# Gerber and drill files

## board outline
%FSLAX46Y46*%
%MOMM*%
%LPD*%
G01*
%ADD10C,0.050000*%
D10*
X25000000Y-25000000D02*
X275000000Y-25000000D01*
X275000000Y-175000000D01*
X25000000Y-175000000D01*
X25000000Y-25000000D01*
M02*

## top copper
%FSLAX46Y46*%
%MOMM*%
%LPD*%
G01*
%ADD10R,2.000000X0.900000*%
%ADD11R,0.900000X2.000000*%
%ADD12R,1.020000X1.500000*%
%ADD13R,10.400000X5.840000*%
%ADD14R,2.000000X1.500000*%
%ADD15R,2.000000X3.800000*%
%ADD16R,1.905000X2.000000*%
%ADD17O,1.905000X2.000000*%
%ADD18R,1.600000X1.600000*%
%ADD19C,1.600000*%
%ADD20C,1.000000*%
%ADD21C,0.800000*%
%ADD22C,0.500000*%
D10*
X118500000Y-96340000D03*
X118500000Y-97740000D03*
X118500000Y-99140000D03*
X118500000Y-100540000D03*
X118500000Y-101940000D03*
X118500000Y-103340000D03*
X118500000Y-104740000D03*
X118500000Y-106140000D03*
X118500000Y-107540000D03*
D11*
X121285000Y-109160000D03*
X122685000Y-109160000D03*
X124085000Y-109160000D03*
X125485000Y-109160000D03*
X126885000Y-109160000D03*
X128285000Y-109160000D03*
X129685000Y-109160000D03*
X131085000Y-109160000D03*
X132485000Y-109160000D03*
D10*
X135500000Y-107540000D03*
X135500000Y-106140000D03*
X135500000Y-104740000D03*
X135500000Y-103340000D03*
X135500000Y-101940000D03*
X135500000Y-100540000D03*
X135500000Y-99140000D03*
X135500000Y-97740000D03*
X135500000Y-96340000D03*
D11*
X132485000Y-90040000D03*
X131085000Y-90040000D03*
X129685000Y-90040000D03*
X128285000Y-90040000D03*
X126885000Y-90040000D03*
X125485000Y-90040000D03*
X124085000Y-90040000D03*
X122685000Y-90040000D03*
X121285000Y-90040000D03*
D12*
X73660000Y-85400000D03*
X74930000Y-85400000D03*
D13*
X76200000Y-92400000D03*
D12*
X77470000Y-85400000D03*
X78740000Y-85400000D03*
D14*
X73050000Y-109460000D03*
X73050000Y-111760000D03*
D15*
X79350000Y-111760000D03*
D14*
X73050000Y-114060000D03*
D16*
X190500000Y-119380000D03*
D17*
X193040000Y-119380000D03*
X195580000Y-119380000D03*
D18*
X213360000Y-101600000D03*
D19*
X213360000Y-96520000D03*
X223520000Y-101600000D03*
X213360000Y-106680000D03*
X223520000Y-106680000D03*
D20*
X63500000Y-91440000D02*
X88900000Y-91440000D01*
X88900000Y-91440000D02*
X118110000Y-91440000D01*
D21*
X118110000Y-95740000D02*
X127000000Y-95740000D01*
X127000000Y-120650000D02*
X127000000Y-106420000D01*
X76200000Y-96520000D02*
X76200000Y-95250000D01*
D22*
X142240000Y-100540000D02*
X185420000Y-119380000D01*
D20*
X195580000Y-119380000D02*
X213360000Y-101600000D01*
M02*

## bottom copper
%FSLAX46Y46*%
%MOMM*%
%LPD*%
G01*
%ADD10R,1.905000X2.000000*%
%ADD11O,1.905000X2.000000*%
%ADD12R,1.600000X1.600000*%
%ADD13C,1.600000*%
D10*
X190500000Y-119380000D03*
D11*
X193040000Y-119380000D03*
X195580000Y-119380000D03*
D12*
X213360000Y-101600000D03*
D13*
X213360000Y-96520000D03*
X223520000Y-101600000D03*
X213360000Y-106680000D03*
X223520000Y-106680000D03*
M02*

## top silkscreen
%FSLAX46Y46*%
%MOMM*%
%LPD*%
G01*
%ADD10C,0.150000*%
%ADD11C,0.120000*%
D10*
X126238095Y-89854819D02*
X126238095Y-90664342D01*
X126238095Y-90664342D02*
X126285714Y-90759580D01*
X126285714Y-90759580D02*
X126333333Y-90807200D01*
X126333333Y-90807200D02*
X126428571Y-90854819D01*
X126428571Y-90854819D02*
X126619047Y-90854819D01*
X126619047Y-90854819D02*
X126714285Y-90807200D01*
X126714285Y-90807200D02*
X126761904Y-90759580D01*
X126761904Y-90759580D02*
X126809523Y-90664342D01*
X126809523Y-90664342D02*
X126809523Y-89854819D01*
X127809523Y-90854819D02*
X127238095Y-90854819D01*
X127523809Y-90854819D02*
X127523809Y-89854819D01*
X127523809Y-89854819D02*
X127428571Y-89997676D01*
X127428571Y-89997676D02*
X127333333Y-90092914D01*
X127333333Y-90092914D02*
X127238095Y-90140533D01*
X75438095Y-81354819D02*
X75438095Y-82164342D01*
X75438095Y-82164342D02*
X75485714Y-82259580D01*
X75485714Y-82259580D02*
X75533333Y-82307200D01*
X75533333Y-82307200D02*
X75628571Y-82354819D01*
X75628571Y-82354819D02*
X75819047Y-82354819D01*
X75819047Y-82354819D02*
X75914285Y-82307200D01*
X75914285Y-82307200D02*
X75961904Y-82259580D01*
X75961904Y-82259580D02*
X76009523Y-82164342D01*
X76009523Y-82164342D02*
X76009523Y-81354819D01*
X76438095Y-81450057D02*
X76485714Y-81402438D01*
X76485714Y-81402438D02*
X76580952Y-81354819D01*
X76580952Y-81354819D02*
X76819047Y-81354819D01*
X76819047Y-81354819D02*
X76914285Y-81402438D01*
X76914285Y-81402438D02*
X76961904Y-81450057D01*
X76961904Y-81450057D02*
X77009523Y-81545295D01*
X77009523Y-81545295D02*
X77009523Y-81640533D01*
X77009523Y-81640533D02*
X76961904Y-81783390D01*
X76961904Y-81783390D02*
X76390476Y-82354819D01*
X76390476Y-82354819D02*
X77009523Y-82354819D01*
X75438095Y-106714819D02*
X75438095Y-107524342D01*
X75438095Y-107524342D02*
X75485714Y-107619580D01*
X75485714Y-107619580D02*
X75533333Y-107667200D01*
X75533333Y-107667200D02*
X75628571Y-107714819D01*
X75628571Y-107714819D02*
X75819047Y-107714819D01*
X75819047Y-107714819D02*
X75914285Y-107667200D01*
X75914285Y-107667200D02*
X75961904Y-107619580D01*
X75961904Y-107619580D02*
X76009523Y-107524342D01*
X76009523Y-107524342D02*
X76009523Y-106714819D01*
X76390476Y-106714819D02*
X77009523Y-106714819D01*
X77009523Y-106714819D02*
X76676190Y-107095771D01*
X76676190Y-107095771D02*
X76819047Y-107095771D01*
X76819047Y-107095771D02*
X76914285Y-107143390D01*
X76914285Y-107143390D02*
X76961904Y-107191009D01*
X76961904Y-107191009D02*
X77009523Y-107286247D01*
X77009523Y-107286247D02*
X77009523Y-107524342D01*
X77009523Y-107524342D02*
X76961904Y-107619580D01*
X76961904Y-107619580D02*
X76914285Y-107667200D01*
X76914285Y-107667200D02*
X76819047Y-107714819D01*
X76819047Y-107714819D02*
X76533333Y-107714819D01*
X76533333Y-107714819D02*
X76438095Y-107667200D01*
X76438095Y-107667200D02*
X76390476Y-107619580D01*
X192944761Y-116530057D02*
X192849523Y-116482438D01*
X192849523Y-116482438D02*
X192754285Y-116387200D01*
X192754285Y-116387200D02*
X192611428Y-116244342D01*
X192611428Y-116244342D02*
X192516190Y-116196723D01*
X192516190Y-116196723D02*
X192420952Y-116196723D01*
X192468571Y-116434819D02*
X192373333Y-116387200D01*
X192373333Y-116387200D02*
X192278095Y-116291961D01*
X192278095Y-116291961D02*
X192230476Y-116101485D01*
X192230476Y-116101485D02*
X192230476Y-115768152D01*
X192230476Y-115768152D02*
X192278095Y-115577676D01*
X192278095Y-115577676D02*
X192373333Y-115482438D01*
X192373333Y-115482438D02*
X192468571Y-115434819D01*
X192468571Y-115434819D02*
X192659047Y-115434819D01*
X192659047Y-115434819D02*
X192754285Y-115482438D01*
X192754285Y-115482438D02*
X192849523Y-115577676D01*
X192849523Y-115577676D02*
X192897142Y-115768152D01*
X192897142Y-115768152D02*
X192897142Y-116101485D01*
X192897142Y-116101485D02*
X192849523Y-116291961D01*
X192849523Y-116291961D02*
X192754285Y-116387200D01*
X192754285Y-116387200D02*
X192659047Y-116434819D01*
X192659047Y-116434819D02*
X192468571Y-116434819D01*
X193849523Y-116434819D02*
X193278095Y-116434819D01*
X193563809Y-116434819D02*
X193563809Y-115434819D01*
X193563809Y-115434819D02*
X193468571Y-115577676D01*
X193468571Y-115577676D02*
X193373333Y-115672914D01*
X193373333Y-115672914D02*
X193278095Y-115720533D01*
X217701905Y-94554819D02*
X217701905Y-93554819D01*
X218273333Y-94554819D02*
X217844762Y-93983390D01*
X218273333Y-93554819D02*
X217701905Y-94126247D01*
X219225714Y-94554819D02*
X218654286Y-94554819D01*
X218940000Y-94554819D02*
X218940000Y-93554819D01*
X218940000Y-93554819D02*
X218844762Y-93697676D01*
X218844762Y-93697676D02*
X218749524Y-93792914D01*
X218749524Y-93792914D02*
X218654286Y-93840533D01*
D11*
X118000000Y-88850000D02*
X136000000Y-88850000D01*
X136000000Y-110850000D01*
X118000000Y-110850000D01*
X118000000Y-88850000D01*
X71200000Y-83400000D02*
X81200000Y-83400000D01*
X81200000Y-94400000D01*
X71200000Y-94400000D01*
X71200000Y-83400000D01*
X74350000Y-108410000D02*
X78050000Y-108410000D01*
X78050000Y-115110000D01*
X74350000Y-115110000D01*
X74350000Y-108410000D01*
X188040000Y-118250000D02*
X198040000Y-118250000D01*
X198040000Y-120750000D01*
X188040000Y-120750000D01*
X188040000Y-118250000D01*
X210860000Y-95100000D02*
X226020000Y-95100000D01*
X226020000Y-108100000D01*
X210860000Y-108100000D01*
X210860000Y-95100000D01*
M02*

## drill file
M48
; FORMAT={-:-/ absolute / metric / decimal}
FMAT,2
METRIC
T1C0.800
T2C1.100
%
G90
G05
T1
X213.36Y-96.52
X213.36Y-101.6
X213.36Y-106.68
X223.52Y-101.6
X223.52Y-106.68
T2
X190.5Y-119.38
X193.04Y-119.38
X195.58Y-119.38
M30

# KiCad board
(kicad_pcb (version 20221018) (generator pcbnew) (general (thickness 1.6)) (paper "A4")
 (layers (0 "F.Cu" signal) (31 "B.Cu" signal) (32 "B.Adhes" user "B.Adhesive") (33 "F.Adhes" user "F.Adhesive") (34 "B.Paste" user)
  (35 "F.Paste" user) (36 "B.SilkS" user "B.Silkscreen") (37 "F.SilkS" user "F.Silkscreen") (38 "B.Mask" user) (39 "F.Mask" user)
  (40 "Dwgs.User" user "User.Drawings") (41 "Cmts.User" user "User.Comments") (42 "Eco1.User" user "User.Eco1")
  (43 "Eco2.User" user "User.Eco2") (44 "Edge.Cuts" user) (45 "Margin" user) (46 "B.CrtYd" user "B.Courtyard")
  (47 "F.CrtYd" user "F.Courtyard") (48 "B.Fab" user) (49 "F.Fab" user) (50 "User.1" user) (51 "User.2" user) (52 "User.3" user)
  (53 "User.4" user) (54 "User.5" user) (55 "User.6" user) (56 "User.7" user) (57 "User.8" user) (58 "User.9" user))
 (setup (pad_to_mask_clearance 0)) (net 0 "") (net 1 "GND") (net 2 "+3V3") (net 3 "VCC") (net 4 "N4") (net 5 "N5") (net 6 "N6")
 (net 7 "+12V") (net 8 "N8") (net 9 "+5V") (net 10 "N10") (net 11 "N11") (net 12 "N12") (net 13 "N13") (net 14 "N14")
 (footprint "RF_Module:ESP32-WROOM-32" (layer "F.Cu") (at 127 101.6)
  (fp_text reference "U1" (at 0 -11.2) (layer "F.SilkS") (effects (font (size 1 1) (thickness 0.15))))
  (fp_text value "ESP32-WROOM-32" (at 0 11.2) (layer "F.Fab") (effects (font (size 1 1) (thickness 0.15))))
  (fp_rect (start -9 -12.75) (end 9 9.25) (stroke (width 0.12) (type solid)) (fill none) (layer "F.SilkS"))
  (pad "1" smd rect (at -8.5 -5.26) (size 2 0.9) (layers "F.Cu" "F.Paste" "F.Mask") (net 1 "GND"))
  (pad "2" smd rect (at -8.5 -3.86) (size 2 0.9) (layers "F.Cu" "F.Paste" "F.Mask") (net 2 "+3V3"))
  (pad "3" smd rect (at -8.5 -2.46) (size 2 0.9) (layers "F.Cu" "F.Paste" "F.Mask") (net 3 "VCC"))
  (pad "4" smd rect (at -8.5 -1.06) (size 2 0.9) (layers "F.Cu" "F.Paste" "F.Mask") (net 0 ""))
  (pad "5" smd rect (at -8.5 0.34) (size 2 0.9) (layers "F.Cu" "F.Paste" "F.Mask") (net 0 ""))
  (pad "6" smd rect (at -8.5 1.74) (size 2 0.9) (layers "F.Cu" "F.Paste" "F.Mask") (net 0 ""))
  (pad "7" smd rect (at -8.5 3.14) (size 2 0.9) (layers "F.Cu" "F.Paste" "F.Mask") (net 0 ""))
  (pad "8" smd rect (at -8.5 4.54) (size 2 0.9) (layers "F.Cu" "F.Paste" "F.Mask") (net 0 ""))
  (pad "9" smd rect (at -8.5 5.94) (size 2 0.9) (layers "F.Cu" "F.Paste" "F.Mask") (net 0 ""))
  (pad "10" smd rect (at -5.715 7.56) (size 0.9 2) (layers "F.Cu" "F.Paste" "F.Mask") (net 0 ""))
  (pad "11" smd rect (at -4.315 7.56) (size 0.9 2) (layers "F.Cu" "F.Paste" "F.Mask") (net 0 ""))
  (pad "12" smd rect (at -2.915 7.56) (size 0.9 2) (layers "F.Cu" "F.Paste" "F.Mask") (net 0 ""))
  (pad "13" smd rect (at -1.515 7.56) (size 0.9 2) (layers "F.Cu" "F.Paste" "F.Mask") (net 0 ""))
  (pad "14" smd rect (at -0.115 7.56) (size 0.9 2) (layers "F.Cu" "F.Paste" "F.Mask") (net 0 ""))
  (pad "15" smd rect (at 1.285 7.56) (size 0.9 2) (layers "F.Cu" "F.Paste" "F.Mask") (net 1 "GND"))
  (pad "16" smd rect (at 2.685 7.56) (size 0.9 2) (layers "F.Cu" "F.Paste" "F.Mask") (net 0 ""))
  (pad "17" smd rect (at 4.085 7.56) (size 0.9 2) (layers "F.Cu" "F.Paste" "F.Mask") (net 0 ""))
  (pad "18" smd rect (at 5.485 7.56) (size 0.9 2) (layers "F.Cu" "F.Paste" "F.Mask") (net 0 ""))
  (pad "19" smd rect (at 8.5 5.94) (size 2 0.9) (layers "F.Cu" "F.Paste" "F.Mask") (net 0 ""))
  (pad "20" smd rect (at 8.5 4.54) (size 2 0.9) (layers "F.Cu" "F.Paste" "F.Mask") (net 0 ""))
  (pad "21" smd rect (at 8.5 3.14) (size 2 0.9) (layers "F.Cu" "F.Paste" "F.Mask") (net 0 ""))
  (pad "22" smd rect (at 8.5 1.74) (size 2 0.9) (layers "F.Cu" "F.Paste" "F.Mask") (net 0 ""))
  (pad "23" smd rect (at 8.5 0.34) (size 2 0.9) (layers "F.Cu" "F.Paste" "F.Mask") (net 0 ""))
  (pad "24" smd rect (at 8.5 -1.06) (size 2 0.9) (layers "F.Cu" "F.Paste" "F.Mask") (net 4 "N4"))
  (pad "25" smd rect (at 8.5 -2.46) (size 2 0.9) (layers "F.Cu" "F.Paste" "F.Mask") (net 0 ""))
  (pad "26" smd rect (at 8.5 -3.86) (size 2 0.9) (layers "F.Cu" "F.Paste" "F.Mask") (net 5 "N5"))
  (pad "27" smd rect (at 8.5 -5.26) (size 2 0.9) (layers "F.Cu" "F.Paste" "F.Mask") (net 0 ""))
  (pad "28" smd rect (at 5.485 -11.56) (size 0.9 2) (layers "F.Cu" "F.Paste" "F.Mask") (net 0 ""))
  (pad "29" smd rect (at 4.085 -11.56) (size 0.9 2) (layers "F.Cu" "F.Paste" "F.Mask") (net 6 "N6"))
  (pad "30" smd rect (at 2.685 -11.56) (size 0.9 2) (layers "F.Cu" "F.Paste" "F.Mask") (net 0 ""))
  (pad "31" smd rect (at 1.285 -11.56) (size 0.9 2) (layers "F.Cu" "F.Paste" "F.Mask") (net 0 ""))
  (pad "32" smd rect (at -0.115 -11.56) (size 0.9 2) (layers "F.Cu" "F.Paste" "F.Mask") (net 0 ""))
  (pad "33" smd rect (at -1.515 -11.56) (size 0.9 2) (layers "F.Cu" "F.Paste" "F.Mask") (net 3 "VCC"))
  (pad "34" smd rect (at -2.915 -11.56) (size 0.9 2) (layers "F.Cu" "F.Paste" "F.Mask") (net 3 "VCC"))
  (pad "35" smd rect (at -4.315 -11.56) (size 0.9 2) (layers "F.Cu" "F.Paste" "F.Mask") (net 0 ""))
  (pad "36" smd rect (at -5.715 -11.56) (size 0.9 2) (layers "F.Cu" "F.Paste" "F.Mask") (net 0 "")))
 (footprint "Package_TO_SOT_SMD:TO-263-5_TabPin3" (layer "F.Cu") (at 76.2 88.9)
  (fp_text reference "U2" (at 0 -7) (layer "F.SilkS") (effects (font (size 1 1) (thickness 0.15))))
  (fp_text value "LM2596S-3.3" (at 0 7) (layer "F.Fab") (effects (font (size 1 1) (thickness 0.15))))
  (fp_rect (start -5 -5.5) (end 5 5.5) (stroke (width 0.12) (type solid)) (fill none) (layer "F.SilkS"))
  (pad "1" smd rect (at -2.54 -3.5) (size 1.02 1.5) (layers "F.Cu" "F.Paste" "F.Mask") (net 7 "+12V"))
  (pad "2" smd rect (at -1.27 -3.5) (size 1.02 1.5) (layers "F.Cu" "F.Paste" "F.Mask") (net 2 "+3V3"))
  (pad "3" smd rect (at 0 3.5) (size 10.4 5.84) (layers "F.Cu" "F.Paste" "F.Mask") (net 1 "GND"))
  (pad "4" smd rect (at 1.27 -3.5) (size 1.02 1.5) (layers "F.Cu" "F.Paste" "F.Mask") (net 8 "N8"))
  (pad "5" smd rect (at 2.54 -3.5) (size 1.02 1.5) (layers "F.Cu" "F.Paste" "F.Mask") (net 7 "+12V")))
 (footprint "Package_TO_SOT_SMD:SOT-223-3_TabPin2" (layer "F.Cu") (at 76.2 111.76)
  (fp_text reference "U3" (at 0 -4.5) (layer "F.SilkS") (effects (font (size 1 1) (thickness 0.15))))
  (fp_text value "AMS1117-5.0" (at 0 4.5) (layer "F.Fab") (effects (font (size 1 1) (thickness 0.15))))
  (fp_rect (start -1.85 -3.35) (end 1.85 3.35) (stroke (width 0.12) (type solid)) (fill none) (layer "F.SilkS"))
  (pad "1" smd rect (at -3.15 -2.3) (size 2 1.5) (layers "F.Cu" "F.Paste" "F.Mask") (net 1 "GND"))
  (pad "2" smd rect (at -3.15 0) (size 2 1.5) (layers "F.Cu" "F.Paste" "F.Mask") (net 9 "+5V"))
  (pad "2" smd rect (at 3.15 0) (size 2 3.8) (layers "F.Cu" "F.Paste" "F.Mask") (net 9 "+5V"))
  (pad "3" smd rect (at -3.15 2.3) (size 2 1.5) (layers "F.Cu" "F.Paste" "F.Mask") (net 2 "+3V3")))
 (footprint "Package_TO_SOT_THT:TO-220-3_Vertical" (layer "F.Cu") (at 190.5 119.38)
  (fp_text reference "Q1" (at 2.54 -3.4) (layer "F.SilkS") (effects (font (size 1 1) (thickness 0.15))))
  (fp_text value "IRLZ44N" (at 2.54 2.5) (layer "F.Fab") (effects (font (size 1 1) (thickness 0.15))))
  (fp_rect (start -2.46 -1.13) (end 7.54 1.37) (stroke (width 0.12) (type solid)) (fill none) (layer "F.SilkS"))
  (pad "1" thru_hole rect (at 0 0) (size 1.905 2) (drill 1.1) (layers "*.Cu" "*.Mask") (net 6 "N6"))
  (pad "2" thru_hole oval (at 2.54 0) (size 1.905 2) (drill 1.1) (layers "*.Cu" "*.Mask") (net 1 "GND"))
  (pad "3" thru_hole oval (at 5.08 0) (size 1.905 2) (drill 1.1) (layers "*.Cu" "*.Mask") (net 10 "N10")))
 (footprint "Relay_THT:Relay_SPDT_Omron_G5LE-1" (layer "F.Cu") (at 213.36 101.6)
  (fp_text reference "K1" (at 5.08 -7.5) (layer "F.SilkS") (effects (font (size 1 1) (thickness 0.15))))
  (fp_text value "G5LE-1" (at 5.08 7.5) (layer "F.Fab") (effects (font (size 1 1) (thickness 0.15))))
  (fp_rect (start -2.5 -6.5) (end 12.66 6.5) (stroke (width 0.12) (type solid)) (fill none) (layer "F.SilkS"))
  (pad "1" thru_hole rect (at 0 0) (size 1.6 1.6) (drill 0.8) (layers "*.Cu" "*.Mask") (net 10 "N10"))
  (pad "2" thru_hole circle (at 0 -5.08) (size 1.6 1.6) (drill 0.8) (layers "*.Cu" "*.Mask") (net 9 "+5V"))
  (pad "4" thru_hole circle (at 10.16 0) (size 1.6 1.6) (drill 0.8) (layers "*.Cu" "*.Mask") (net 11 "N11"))
  (pad "5" thru_hole circle (at 0 5.08) (size 1.6 1.6) (drill 0.8) (layers "*.Cu" "*.Mask") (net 1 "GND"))
  (pad "8" thru_hole circle (at 10.16 5.08) (size 1.6 1.6) (drill 0.8) (layers "*.Cu" "*.Mask") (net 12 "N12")))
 (gr_rect (start 25 25) (end 275 175) (stroke (width 0.05) (type solid)) (fill none) (layer "Edge.Cuts"))
 (segment (start 63.5 91.44) (end 88.9 91.44) (width 1.0) (layer "F.Cu") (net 7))
 (segment (start 88.9 91.44) (end 118.11 91.44) (width 1.0) (layer "F.Cu") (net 2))
 (segment (start 118.11 95.74) (end 127 95.74) (width 0.8) (layer "F.Cu") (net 2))
 (segment (start 127 120.65) (end 127 106.42) (width 0.8) (layer "F.Cu") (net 1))
 (segment (start 76.2 96.52) (end 76.2 95.25) (width 0.8) (layer "F.Cu") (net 1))
 (segment (start 142.24 100.54) (end 185.42 119.38) (width 0.5) (layer "F.Cu") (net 6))
 (segment (start 195.58 119.38) (end 213.36 101.6) (width 1.0) (layer "F.Cu") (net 10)))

